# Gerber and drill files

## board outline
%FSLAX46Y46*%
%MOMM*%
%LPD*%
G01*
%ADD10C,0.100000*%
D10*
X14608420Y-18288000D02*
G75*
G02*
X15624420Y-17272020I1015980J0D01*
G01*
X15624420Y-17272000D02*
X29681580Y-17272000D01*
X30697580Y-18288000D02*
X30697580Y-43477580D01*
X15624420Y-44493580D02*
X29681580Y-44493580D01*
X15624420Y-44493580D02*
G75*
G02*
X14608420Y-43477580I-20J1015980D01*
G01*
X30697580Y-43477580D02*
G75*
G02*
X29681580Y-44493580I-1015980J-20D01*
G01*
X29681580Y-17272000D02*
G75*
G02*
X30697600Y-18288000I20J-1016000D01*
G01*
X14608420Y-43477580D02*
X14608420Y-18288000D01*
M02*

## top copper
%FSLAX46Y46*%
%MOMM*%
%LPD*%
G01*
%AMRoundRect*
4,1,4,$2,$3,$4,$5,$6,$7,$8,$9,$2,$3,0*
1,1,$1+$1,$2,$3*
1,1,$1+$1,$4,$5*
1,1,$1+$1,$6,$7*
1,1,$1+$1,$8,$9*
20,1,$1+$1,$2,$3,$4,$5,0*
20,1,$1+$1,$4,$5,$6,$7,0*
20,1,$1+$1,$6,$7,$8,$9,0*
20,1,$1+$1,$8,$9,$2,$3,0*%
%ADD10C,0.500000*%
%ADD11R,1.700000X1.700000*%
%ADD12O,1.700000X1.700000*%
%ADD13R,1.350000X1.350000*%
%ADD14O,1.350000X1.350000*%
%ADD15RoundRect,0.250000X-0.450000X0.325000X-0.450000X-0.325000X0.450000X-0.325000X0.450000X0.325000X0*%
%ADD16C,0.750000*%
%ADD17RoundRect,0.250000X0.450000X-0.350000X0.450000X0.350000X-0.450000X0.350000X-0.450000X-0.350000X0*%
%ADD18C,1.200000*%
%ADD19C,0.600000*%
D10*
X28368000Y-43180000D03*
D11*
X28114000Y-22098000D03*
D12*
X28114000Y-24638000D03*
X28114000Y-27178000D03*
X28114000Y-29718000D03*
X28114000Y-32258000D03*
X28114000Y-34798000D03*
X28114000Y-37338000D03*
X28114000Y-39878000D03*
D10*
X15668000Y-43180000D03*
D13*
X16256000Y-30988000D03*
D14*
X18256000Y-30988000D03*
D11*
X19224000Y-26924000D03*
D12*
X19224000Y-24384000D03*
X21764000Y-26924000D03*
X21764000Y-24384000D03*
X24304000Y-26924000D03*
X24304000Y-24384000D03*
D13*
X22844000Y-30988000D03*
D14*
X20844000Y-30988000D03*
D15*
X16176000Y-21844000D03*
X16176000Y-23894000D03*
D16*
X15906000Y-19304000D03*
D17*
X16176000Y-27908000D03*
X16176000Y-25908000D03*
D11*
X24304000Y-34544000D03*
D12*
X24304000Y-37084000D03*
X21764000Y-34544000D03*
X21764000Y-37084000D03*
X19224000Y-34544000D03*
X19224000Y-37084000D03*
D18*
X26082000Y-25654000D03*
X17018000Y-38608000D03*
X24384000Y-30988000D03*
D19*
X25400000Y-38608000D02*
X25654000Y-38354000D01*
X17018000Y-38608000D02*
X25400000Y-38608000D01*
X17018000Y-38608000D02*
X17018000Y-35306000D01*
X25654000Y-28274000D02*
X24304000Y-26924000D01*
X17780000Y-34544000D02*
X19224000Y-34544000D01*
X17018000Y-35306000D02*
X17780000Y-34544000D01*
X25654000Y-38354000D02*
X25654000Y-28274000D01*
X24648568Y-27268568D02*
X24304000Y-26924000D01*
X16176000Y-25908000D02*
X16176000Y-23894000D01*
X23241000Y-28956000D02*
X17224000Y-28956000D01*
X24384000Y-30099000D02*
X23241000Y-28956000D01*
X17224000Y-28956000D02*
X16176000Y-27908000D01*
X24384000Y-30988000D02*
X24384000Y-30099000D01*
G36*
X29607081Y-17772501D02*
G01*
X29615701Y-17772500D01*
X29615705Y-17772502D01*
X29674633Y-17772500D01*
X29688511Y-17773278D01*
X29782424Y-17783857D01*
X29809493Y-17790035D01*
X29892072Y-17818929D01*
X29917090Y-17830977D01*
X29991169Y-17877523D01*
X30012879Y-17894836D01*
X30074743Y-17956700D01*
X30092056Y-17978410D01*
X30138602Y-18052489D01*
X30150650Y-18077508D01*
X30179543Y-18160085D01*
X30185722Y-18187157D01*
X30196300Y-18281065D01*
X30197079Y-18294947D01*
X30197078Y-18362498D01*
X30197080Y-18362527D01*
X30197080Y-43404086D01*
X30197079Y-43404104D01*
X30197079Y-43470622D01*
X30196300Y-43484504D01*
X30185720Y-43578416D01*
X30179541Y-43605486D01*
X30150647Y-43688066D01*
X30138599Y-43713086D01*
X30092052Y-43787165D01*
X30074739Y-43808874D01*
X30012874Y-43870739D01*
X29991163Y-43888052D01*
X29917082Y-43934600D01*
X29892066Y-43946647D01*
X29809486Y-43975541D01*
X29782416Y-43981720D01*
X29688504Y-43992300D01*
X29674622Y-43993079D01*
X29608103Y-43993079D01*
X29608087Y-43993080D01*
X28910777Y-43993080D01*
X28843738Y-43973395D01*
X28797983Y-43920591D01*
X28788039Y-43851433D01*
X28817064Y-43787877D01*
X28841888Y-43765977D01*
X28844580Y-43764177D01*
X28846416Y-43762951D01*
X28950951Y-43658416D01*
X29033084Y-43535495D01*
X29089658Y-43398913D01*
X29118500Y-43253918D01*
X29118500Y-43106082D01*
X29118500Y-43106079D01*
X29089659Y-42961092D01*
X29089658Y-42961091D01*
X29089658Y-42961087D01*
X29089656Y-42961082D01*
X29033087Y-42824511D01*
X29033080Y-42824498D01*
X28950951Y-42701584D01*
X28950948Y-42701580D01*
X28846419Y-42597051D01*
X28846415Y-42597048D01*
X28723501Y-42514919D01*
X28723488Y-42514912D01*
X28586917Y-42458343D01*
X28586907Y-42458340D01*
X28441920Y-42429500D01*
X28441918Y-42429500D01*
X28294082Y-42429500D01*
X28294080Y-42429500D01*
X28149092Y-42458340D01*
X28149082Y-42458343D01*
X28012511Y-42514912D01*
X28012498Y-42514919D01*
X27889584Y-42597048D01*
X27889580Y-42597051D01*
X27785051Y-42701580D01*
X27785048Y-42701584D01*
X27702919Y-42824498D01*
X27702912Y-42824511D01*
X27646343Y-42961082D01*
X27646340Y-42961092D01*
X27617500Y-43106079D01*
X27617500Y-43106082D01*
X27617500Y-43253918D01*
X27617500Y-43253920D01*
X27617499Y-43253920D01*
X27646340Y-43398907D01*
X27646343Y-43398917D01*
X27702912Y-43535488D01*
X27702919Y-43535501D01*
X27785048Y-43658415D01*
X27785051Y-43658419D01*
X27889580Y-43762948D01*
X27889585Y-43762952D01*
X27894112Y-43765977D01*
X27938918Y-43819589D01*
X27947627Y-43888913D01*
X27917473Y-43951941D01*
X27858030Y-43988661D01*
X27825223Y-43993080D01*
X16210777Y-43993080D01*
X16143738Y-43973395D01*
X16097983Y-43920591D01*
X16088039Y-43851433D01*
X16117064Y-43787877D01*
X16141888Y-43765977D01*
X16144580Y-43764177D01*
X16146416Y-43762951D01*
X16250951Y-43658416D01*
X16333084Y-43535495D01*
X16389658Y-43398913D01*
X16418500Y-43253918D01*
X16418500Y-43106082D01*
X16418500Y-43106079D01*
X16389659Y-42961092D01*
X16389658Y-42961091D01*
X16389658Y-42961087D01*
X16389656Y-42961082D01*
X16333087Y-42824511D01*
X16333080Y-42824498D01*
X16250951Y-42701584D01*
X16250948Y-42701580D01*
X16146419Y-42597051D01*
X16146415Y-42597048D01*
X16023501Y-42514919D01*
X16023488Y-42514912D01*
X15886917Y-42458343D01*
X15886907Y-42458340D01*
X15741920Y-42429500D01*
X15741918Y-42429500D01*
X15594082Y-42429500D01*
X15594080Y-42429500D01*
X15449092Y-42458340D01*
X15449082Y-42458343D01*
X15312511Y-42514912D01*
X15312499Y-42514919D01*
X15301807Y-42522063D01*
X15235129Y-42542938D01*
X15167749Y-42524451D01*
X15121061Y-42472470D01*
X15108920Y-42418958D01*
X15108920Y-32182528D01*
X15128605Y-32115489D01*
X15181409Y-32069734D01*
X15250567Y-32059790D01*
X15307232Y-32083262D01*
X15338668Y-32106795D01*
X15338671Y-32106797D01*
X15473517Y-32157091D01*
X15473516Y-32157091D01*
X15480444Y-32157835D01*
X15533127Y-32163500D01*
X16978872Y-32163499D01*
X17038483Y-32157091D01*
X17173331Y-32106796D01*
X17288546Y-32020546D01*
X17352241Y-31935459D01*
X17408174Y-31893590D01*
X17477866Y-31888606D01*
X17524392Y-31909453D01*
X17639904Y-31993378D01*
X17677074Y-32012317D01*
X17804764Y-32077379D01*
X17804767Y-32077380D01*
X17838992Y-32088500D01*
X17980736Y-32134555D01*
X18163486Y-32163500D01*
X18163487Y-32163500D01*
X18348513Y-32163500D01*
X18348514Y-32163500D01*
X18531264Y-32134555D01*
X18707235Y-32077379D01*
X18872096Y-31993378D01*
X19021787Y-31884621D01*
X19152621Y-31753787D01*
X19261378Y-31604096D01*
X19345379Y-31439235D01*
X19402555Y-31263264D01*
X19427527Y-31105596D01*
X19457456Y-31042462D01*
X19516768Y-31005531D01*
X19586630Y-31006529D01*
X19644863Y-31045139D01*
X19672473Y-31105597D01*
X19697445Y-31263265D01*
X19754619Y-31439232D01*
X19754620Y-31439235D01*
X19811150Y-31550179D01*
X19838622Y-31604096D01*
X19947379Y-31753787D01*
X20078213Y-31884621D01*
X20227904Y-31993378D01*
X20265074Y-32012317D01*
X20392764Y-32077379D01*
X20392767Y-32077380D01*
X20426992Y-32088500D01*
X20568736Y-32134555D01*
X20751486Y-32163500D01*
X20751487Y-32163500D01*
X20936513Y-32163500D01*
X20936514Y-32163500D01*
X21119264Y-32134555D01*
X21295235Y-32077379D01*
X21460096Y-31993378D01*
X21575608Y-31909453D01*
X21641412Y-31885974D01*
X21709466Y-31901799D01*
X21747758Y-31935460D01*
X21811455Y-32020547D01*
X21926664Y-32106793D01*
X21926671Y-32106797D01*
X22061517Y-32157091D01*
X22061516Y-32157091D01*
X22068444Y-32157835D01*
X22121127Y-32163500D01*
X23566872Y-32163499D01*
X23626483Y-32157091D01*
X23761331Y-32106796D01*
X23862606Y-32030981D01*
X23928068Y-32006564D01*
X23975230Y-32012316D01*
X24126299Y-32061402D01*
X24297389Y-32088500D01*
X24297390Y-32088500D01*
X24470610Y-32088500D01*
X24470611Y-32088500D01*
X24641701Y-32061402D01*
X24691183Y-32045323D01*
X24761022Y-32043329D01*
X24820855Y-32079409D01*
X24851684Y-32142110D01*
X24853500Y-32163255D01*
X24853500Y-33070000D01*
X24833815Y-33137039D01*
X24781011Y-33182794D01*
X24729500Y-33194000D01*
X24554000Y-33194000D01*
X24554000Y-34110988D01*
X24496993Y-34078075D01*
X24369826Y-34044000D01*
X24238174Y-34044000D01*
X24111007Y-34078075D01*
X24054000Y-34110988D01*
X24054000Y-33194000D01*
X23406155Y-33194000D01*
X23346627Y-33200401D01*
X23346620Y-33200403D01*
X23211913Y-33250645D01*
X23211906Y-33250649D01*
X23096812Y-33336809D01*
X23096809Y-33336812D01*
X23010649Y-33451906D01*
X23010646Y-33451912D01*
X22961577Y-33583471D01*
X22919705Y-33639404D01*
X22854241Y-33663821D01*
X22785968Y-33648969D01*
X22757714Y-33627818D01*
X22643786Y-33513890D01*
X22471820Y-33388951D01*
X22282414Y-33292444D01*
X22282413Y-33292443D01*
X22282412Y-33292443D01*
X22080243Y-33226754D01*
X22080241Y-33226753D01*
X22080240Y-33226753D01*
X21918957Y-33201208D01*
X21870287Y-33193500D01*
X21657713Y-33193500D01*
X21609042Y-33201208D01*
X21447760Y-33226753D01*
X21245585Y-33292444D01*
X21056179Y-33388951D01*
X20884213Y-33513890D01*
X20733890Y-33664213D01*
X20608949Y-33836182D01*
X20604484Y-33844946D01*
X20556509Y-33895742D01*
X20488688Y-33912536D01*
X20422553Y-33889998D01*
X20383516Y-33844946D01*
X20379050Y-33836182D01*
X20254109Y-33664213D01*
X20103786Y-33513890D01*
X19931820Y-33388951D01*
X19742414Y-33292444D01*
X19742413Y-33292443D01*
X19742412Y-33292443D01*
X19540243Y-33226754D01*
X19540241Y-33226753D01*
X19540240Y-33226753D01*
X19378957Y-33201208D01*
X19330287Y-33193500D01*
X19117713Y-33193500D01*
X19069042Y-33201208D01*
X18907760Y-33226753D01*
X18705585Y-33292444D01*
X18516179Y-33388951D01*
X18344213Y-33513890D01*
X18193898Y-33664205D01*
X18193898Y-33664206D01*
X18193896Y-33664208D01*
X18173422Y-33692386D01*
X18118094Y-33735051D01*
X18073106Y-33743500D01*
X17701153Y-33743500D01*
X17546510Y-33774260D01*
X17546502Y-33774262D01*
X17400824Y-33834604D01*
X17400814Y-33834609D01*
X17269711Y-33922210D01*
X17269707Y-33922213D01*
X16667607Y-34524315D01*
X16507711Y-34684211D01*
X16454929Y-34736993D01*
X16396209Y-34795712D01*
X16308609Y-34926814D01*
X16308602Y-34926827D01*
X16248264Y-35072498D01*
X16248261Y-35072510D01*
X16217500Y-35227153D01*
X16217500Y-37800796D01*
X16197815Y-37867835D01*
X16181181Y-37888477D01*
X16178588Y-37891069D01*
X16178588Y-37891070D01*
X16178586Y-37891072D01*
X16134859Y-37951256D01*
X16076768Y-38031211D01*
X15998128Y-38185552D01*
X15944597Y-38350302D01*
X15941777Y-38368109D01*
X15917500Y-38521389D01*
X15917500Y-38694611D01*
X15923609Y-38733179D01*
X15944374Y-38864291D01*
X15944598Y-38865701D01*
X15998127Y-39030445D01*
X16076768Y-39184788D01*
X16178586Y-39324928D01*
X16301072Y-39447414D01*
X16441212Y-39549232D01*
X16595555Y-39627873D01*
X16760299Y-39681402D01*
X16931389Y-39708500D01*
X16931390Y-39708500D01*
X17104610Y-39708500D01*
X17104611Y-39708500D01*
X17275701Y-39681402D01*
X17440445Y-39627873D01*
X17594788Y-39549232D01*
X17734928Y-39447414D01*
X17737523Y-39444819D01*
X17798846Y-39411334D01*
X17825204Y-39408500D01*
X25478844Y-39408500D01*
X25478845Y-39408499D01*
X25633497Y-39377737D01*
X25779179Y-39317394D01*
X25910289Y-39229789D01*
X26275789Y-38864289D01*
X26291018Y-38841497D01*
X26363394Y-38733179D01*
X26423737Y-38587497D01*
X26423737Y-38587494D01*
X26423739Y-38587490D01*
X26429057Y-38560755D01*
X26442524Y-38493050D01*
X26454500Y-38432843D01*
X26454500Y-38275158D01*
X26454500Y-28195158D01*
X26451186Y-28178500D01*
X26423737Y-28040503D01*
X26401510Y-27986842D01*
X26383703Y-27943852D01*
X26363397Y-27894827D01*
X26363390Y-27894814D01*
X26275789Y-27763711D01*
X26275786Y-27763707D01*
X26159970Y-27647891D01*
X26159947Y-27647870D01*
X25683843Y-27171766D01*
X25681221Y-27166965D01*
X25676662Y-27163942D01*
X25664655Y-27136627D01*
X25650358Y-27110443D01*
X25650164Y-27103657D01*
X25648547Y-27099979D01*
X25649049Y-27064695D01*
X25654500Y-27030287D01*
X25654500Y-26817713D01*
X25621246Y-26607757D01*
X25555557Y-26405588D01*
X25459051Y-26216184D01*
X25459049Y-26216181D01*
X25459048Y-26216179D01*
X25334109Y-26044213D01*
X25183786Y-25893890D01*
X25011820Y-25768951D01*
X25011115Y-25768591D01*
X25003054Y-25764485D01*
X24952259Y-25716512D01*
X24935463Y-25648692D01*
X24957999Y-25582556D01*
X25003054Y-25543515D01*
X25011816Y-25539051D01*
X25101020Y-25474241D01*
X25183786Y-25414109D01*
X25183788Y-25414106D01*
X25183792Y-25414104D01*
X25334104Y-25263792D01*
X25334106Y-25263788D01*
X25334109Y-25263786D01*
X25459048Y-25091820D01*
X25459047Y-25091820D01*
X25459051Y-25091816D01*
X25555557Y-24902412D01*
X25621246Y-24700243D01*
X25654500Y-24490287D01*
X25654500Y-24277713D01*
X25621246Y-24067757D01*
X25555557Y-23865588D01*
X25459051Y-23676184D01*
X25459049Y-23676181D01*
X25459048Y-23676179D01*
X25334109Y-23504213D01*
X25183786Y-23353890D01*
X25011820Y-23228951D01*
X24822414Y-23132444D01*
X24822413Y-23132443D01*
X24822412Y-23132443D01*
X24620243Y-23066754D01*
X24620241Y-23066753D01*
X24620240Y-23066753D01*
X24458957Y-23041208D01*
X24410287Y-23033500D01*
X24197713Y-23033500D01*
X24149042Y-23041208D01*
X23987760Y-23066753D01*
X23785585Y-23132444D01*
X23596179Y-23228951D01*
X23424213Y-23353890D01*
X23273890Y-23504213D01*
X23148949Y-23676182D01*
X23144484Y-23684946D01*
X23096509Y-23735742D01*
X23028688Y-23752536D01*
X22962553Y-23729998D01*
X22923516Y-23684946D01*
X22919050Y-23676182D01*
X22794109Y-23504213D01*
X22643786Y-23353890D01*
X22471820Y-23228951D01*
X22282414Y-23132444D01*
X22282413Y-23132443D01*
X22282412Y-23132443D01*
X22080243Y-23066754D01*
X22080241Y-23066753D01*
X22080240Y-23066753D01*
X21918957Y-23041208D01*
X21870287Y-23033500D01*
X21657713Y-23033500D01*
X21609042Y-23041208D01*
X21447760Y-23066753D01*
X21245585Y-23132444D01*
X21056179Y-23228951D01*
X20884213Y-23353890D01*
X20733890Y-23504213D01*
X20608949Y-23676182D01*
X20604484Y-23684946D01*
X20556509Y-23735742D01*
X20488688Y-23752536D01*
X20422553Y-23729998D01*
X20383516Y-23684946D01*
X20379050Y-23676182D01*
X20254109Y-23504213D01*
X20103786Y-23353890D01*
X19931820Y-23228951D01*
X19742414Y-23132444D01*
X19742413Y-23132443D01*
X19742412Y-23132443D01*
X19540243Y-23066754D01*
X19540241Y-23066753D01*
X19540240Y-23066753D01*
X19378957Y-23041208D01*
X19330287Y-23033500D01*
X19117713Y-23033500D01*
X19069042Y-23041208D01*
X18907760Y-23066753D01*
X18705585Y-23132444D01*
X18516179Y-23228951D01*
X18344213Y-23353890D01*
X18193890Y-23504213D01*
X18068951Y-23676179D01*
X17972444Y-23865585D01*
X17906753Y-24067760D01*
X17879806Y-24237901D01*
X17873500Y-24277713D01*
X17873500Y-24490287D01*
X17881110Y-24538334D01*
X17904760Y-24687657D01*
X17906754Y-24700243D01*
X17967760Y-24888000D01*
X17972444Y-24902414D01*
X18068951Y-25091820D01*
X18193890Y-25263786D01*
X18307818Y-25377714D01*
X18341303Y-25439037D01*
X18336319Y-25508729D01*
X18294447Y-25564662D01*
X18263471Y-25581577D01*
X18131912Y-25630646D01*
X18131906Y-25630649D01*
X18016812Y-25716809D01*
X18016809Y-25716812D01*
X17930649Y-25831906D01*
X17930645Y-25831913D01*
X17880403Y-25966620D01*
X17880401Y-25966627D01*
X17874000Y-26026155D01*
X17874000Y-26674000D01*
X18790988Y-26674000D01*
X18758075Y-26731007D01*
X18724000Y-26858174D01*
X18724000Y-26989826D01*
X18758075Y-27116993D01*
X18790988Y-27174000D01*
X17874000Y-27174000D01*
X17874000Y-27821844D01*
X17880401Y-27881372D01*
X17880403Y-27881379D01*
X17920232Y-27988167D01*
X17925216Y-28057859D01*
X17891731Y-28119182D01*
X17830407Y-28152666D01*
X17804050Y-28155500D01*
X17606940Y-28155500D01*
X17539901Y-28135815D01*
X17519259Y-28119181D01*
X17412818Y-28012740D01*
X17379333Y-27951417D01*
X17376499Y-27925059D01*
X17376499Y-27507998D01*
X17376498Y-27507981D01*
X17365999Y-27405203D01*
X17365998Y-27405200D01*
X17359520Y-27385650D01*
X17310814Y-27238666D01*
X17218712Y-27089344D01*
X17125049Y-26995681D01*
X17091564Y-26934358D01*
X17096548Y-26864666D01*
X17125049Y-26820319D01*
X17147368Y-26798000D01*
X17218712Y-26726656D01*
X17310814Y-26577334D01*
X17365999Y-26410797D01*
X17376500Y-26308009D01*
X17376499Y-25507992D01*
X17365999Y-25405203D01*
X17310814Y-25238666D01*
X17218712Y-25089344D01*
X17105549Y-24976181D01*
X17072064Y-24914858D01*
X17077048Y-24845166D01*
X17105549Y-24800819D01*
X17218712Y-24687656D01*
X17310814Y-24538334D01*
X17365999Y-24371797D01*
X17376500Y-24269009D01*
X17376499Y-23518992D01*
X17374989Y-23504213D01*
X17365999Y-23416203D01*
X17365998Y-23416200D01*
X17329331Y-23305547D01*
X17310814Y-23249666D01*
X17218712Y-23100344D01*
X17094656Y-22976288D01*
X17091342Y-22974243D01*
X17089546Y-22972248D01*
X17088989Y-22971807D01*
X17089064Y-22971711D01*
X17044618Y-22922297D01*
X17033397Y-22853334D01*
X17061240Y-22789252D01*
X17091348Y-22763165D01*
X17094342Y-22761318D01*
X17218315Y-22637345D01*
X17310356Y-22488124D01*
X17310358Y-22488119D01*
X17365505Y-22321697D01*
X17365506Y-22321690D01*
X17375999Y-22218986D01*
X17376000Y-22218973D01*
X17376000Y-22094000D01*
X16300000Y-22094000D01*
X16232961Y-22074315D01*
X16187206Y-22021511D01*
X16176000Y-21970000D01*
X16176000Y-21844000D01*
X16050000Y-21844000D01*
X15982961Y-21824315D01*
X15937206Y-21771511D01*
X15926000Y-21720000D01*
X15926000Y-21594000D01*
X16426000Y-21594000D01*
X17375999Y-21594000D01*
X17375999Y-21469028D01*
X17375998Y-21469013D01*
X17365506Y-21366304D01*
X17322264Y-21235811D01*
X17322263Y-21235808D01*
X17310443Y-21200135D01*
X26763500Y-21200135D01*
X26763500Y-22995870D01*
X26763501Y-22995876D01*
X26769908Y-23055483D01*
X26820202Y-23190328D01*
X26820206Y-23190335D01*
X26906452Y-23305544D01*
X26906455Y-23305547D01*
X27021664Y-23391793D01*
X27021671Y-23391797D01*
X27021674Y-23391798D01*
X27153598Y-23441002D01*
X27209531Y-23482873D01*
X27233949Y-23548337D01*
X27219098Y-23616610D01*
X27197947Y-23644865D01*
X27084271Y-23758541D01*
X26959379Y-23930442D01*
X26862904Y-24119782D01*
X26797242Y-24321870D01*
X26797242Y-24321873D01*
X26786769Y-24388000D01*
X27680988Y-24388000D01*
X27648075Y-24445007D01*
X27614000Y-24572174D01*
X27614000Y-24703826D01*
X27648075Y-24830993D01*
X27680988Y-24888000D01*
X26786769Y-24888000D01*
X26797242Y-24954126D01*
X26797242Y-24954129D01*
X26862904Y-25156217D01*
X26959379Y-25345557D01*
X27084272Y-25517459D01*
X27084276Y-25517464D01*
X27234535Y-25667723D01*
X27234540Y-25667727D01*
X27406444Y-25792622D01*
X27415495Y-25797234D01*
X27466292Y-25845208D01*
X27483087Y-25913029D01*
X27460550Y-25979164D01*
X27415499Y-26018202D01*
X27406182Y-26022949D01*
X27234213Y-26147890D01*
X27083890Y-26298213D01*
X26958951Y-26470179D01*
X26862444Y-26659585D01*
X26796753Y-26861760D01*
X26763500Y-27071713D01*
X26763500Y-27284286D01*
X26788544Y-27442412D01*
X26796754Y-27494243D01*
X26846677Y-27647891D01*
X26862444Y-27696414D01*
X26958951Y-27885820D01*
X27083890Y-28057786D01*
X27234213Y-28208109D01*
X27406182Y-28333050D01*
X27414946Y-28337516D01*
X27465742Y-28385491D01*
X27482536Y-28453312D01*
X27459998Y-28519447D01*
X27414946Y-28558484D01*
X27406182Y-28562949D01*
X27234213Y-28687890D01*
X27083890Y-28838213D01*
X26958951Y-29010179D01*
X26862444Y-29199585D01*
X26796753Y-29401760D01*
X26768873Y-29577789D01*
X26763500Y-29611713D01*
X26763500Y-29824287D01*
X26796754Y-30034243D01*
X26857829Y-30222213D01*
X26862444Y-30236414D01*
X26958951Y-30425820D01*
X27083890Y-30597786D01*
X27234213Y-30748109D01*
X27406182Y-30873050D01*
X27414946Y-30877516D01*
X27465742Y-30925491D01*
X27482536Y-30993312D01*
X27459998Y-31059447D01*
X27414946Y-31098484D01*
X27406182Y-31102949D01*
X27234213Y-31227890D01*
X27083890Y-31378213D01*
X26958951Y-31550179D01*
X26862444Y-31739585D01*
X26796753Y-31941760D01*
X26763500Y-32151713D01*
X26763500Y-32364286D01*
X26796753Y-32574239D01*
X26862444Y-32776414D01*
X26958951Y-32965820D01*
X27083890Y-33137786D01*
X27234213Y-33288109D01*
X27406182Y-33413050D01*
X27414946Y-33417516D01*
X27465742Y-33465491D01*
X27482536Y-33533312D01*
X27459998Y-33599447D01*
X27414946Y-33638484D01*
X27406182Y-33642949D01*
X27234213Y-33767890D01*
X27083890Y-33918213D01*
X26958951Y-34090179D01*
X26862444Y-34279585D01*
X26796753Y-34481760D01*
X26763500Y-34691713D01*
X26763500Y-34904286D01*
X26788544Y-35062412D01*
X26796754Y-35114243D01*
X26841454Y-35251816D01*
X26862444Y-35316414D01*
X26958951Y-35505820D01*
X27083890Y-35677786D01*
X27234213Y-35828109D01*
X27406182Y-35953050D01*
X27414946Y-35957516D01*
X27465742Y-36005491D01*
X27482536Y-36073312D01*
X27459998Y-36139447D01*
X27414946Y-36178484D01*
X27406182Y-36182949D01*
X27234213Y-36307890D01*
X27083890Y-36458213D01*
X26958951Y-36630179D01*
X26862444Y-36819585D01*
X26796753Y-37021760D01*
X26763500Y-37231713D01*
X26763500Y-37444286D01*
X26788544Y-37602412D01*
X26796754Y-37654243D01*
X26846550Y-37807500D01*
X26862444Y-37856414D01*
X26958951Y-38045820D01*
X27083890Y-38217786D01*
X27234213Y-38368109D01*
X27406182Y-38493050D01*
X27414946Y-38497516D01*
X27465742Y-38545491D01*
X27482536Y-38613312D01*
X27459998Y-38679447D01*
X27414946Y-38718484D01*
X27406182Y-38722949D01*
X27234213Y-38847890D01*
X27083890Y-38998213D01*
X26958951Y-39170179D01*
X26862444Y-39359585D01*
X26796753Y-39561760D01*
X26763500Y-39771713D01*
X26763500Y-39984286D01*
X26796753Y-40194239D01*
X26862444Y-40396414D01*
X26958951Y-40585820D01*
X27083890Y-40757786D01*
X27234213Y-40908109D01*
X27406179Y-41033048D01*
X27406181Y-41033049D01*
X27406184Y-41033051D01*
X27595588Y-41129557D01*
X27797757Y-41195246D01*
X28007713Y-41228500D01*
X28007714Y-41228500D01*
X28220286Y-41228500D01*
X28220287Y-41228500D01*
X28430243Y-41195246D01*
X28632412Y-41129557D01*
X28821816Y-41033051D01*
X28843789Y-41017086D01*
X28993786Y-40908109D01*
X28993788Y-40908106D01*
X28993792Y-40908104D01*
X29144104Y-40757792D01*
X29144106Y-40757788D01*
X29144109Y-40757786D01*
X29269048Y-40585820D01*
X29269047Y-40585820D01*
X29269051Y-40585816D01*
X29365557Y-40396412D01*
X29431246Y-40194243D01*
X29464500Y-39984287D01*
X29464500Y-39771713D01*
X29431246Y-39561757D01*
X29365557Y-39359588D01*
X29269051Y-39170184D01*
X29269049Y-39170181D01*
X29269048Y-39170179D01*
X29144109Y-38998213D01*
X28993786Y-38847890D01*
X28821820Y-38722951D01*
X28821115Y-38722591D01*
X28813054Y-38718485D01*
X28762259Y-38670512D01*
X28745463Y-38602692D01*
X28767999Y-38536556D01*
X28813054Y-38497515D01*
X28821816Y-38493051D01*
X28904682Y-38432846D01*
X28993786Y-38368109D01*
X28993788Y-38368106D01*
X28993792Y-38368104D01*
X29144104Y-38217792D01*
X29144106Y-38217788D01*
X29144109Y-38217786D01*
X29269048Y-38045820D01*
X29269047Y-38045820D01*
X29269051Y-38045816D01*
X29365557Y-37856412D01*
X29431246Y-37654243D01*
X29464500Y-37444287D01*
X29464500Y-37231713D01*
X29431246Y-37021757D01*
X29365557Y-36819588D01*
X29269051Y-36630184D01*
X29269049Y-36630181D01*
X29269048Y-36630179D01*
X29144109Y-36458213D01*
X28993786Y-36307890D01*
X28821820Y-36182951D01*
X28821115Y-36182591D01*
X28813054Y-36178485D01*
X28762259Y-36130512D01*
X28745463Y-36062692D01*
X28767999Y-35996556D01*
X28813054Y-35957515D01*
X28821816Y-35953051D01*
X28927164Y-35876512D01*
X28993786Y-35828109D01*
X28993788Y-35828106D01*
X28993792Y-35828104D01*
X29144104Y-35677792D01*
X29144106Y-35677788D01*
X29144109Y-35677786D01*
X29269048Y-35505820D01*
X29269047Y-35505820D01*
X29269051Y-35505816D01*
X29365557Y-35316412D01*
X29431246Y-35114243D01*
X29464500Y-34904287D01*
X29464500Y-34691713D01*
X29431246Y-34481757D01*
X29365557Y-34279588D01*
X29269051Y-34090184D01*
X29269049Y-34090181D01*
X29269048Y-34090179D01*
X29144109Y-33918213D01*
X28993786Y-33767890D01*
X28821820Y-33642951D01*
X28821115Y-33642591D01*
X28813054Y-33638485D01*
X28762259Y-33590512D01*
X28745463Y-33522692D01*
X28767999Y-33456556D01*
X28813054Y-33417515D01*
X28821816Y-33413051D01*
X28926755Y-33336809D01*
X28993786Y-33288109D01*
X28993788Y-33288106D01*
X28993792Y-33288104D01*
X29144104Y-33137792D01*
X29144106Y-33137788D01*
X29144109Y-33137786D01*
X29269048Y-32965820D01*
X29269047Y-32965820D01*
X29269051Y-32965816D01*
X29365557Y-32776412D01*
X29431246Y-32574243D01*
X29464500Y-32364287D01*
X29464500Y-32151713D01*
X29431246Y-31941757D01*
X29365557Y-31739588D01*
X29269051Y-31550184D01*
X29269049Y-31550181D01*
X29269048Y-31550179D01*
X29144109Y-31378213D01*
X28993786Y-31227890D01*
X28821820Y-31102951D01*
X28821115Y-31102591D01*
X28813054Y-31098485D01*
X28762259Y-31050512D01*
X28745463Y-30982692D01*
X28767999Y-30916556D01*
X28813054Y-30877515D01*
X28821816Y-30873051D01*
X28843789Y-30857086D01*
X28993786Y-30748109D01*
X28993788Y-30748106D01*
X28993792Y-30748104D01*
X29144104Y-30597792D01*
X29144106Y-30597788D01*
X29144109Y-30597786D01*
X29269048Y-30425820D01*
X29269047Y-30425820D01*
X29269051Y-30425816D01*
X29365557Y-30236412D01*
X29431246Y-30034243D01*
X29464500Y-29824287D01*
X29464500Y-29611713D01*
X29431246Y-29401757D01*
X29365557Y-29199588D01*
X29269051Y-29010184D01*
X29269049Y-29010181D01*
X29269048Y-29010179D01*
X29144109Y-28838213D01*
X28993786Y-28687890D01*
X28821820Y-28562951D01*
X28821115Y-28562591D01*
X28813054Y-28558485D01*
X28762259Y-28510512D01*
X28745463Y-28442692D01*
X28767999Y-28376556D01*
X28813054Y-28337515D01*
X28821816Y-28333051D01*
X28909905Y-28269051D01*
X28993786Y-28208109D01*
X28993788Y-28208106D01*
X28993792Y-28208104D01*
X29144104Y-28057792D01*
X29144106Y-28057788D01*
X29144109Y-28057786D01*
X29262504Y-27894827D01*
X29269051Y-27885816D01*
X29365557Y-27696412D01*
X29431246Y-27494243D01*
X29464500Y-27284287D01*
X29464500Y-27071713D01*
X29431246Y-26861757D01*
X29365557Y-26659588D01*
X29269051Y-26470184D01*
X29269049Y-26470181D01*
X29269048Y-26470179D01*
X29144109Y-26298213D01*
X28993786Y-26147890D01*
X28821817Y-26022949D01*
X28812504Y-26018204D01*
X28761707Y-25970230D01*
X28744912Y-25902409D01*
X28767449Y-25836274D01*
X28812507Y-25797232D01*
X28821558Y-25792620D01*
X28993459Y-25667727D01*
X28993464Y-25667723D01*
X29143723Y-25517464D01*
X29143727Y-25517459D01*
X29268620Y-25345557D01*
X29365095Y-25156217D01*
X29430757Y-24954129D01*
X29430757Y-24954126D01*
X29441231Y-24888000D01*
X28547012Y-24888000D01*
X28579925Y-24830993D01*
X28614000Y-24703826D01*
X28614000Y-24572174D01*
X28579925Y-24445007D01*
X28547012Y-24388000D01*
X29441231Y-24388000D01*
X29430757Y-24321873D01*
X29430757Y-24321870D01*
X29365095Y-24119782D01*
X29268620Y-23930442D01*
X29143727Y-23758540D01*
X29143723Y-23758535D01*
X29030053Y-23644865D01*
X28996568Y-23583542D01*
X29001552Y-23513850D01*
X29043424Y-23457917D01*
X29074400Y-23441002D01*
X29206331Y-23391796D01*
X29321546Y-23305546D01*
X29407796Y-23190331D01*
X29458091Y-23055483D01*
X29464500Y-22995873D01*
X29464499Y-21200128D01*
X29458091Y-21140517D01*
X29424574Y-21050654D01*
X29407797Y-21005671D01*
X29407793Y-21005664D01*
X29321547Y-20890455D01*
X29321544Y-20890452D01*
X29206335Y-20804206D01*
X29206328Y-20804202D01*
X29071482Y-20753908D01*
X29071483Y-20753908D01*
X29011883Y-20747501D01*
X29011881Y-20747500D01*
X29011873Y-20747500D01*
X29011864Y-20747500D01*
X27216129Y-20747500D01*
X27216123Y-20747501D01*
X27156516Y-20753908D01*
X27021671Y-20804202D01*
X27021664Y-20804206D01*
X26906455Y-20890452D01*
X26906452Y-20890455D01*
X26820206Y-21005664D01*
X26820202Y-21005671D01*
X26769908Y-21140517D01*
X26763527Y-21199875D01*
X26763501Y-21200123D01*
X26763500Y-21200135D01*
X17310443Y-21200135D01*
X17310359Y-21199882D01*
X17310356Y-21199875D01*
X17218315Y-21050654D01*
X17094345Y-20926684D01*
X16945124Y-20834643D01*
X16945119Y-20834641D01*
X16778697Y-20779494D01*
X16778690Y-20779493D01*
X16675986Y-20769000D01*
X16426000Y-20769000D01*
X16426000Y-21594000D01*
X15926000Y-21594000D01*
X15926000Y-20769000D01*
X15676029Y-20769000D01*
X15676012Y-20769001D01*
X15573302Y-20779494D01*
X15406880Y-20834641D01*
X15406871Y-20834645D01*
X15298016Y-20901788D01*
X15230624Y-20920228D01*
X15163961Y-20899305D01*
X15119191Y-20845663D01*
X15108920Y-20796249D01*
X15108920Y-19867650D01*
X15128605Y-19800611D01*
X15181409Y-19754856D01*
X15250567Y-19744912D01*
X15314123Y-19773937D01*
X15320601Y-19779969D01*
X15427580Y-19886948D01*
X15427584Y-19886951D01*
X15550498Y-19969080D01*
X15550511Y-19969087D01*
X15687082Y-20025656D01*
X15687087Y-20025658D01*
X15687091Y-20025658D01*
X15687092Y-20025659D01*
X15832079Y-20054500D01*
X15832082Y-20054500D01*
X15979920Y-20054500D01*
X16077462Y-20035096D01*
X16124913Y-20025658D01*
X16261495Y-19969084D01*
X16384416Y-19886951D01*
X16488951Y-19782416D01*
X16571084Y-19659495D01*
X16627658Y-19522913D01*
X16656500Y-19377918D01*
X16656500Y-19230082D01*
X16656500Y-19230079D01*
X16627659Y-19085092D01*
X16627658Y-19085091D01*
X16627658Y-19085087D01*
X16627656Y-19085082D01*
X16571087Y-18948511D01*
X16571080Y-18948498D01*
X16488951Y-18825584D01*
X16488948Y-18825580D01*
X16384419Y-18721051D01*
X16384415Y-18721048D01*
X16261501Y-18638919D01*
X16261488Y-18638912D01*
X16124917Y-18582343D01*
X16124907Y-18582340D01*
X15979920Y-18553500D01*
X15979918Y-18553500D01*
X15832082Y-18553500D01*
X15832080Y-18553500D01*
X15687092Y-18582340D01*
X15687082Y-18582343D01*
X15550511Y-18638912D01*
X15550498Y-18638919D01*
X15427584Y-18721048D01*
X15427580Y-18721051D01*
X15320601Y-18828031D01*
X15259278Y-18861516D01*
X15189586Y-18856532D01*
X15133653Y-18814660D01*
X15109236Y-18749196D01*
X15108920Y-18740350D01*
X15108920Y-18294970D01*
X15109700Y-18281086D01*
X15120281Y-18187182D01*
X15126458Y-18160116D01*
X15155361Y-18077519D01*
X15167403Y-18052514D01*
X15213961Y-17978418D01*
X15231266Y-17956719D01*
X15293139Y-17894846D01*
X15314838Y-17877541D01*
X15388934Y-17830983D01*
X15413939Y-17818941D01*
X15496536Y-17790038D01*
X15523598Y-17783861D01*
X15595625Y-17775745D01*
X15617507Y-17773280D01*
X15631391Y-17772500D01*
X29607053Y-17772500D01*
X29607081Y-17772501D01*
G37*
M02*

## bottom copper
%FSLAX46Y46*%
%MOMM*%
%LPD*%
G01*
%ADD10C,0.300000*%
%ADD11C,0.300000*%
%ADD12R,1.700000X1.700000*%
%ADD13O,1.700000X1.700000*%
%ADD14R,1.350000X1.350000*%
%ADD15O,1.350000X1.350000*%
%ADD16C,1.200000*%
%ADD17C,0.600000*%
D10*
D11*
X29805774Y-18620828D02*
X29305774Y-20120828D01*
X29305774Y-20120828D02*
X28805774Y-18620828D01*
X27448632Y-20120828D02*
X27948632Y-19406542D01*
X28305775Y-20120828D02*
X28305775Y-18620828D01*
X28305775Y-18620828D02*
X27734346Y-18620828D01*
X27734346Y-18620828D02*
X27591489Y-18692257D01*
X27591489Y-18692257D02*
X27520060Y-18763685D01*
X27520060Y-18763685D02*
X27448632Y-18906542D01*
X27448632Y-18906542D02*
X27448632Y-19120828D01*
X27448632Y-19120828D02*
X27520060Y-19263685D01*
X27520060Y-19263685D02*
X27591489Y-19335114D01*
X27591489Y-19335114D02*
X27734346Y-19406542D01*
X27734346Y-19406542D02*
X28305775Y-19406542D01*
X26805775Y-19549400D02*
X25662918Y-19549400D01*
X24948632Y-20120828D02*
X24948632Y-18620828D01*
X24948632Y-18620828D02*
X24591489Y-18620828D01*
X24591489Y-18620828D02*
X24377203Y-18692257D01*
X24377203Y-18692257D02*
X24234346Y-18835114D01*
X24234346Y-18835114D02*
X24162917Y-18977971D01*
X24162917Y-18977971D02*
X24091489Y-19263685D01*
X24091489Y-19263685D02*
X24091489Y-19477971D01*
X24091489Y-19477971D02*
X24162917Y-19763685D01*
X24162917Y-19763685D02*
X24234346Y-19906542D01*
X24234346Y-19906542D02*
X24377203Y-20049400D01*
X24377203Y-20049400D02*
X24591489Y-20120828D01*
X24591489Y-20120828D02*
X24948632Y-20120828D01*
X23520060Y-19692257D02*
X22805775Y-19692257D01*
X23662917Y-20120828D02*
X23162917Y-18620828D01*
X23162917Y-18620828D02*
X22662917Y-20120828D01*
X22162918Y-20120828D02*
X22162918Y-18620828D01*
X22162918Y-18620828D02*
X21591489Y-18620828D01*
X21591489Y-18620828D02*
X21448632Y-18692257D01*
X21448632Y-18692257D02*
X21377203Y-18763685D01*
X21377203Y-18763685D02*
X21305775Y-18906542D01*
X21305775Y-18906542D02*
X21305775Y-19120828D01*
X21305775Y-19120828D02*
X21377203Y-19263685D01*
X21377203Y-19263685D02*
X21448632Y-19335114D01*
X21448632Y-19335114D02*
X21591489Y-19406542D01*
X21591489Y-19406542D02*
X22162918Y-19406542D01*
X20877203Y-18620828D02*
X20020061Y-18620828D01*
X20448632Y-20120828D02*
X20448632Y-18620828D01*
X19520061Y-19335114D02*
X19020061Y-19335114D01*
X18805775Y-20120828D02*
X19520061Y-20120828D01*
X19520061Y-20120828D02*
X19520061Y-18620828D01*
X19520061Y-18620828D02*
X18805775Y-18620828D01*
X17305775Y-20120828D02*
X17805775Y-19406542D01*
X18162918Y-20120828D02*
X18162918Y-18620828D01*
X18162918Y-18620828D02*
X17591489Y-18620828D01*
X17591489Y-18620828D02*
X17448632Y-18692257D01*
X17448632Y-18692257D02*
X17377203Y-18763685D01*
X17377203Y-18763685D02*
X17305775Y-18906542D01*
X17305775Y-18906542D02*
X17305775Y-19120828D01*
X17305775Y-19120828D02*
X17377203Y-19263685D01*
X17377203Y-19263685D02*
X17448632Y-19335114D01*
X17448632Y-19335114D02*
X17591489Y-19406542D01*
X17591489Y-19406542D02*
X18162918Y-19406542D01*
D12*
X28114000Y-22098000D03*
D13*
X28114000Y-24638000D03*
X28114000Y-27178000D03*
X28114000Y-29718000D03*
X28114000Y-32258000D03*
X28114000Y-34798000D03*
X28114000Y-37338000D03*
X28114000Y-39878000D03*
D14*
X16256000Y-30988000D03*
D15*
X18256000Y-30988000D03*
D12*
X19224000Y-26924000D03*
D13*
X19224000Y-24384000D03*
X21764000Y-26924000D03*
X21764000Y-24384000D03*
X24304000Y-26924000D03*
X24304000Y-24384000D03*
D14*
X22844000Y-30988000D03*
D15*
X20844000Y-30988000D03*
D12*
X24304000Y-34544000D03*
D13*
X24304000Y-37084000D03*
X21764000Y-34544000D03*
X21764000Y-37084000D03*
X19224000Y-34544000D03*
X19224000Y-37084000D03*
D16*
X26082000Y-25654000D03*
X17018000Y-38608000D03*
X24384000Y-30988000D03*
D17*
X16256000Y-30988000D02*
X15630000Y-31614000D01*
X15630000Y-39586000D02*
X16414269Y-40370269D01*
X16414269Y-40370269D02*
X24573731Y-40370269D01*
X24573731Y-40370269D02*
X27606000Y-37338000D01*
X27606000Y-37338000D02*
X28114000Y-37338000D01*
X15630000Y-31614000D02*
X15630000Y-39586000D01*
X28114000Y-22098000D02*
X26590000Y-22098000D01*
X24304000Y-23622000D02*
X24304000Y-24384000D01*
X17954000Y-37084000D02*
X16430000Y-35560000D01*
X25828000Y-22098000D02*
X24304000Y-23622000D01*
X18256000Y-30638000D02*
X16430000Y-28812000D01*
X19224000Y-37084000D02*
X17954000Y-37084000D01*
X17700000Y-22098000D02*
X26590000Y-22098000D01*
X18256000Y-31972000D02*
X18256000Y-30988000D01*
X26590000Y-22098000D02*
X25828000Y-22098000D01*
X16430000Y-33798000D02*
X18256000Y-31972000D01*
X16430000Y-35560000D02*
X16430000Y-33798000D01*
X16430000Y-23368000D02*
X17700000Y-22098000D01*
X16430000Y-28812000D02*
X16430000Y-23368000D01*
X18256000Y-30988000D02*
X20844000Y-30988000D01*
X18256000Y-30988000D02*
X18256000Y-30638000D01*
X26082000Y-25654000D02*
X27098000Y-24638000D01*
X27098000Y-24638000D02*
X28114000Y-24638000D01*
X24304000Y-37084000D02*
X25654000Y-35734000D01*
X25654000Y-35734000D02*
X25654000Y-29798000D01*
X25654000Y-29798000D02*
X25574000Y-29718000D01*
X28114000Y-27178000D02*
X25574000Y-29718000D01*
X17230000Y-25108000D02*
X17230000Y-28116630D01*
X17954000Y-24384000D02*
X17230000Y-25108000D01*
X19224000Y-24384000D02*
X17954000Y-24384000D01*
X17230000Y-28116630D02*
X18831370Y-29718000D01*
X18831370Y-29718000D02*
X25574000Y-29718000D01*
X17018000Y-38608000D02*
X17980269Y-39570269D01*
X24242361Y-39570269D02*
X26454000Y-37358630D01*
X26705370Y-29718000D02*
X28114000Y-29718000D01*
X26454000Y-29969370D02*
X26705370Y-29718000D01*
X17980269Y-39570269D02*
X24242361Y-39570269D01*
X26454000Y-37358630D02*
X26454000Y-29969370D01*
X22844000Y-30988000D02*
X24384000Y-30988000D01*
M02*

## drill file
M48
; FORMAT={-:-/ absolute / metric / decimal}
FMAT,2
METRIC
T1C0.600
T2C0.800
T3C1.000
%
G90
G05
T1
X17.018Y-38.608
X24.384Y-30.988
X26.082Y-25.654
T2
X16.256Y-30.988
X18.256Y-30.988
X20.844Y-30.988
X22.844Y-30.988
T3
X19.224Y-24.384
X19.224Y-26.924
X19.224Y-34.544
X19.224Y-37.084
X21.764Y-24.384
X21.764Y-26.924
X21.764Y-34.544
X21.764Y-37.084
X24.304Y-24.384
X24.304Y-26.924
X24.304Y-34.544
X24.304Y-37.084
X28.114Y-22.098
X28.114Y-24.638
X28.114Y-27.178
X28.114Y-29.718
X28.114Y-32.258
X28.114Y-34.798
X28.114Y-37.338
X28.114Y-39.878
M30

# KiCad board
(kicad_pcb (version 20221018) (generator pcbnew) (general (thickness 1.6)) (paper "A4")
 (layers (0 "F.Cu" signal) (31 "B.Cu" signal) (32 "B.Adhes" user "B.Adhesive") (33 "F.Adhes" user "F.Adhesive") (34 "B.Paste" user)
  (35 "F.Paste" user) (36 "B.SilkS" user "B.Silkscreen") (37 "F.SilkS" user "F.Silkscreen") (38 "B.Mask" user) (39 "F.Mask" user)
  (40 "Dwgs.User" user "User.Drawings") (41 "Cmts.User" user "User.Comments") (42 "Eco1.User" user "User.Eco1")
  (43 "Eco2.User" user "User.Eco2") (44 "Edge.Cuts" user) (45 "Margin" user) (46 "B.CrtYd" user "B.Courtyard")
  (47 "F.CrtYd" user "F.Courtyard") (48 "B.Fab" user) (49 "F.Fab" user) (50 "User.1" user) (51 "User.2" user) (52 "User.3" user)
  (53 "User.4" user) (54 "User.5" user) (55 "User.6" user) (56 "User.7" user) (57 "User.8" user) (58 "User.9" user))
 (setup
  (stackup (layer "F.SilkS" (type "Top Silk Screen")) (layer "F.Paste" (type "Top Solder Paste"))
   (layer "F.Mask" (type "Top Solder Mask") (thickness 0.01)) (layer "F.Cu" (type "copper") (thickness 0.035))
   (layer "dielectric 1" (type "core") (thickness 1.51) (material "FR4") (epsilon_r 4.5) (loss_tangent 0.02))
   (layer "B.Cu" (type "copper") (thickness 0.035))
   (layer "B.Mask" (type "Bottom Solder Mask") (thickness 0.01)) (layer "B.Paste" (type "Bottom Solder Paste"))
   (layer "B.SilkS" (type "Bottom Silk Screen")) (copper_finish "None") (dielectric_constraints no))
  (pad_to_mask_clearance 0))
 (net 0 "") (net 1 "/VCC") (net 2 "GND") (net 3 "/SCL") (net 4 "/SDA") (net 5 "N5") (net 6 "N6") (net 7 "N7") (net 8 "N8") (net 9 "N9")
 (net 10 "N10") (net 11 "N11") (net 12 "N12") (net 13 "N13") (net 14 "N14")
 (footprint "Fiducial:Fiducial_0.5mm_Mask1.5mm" (layer "F.Cu") (at 28.368 43.18)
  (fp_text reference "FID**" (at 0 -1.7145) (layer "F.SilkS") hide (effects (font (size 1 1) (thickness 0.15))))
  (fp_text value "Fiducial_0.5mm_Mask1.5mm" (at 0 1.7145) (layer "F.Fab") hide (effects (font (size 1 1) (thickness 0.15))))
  (pad "" smd circle (at 0 0) (size 0.5 0.5) (layers "F.Cu" "F.Mask" "Eco1.User") (solder_mask_margin 0.5) (clearance 0.5)))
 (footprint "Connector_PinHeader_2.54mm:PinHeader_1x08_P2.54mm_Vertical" (layer "F.Cu") (at 28.114 22.098)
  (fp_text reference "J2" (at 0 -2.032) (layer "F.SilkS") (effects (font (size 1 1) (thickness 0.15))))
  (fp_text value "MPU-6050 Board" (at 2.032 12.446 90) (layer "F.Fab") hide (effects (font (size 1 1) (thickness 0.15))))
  (pad "1" thru_hole rect (at 0 0) (size 1.7 1.7) (drill 1) (layers "*.Cu" "*.Mask") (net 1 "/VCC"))
  (pad "2" thru_hole oval (at 0 2.54) (size 1.7 1.7) (drill 1) (layers "*.Cu" "*.Mask") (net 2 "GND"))
  (pad "3" thru_hole oval (at 0 5.08) (size 1.7 1.7) (drill 1) (layers "*.Cu" "*.Mask") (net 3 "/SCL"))
  (pad "4" thru_hole oval (at 0 7.62) (size 1.7 1.7) (drill 1) (layers "*.Cu" "*.Mask") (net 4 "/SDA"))
  (pad "5" thru_hole oval (at 0 10.16) (size 1.7 1.7) (drill 1) (layers "*.Cu" "*.Mask") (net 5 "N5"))
  (pad "6" thru_hole oval (at 0 12.7) (size 1.7 1.7) (drill 1) (layers "*.Cu" "*.Mask") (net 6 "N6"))
  (pad "7" thru_hole oval (at 0 15.24) (size 1.7 1.7) (drill 1) (layers "*.Cu" "*.Mask") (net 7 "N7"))
  (pad "8" thru_hole oval (at 0 17.78) (size 1.7 1.7) (drill 1) (layers "*.Cu" "*.Mask") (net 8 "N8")))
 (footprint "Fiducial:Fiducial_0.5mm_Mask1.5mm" (layer "F.Cu") (at 15.668 43.18)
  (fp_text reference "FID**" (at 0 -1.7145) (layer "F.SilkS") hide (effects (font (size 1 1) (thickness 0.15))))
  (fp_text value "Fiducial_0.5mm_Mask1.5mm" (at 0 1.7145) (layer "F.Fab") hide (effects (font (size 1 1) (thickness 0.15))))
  (pad "" smd circle (at 0 0) (size 0.5 0.5) (layers "F.Cu" "F.Mask" "Eco1.User") (solder_mask_margin 0.5) (clearance 0.5)))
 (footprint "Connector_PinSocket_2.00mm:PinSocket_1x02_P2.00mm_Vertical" (layer "F.Cu") (at 16.256 30.988 90)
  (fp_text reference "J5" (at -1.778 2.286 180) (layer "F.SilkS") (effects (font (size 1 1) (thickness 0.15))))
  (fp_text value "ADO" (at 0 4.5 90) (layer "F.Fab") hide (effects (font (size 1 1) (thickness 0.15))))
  (pad "1" thru_hole rect (at 0 0 90) (size 1.35 1.35) (drill 0.8) (layers "*.Cu" "*.Mask") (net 7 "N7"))
  (pad "2" thru_hole oval (at 0 2 90) (size 1.35 1.35) (drill 0.8) (layers "*.Cu" "*.Mask") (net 1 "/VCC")))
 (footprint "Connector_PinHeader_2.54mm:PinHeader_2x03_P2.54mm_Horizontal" (layer "F.Cu") (at 19.224 26.924 90)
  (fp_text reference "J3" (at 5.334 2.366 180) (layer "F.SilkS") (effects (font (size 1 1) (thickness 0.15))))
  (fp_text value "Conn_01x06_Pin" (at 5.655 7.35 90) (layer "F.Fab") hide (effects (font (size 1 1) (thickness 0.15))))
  (pad "1" thru_hole rect (at 0 0 90) (size 1.7 1.7) (drill 1) (layers "*.Cu" "*.Mask") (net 2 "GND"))
  (pad "2" thru_hole oval (at 2.54 0 90) (size 1.7 1.7) (drill 1) (layers "*.Cu" "*.Mask") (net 3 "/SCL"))
  (pad "3" thru_hole oval (at 0 2.54 90) (size 1.7 1.7) (drill 1) (layers "*.Cu" "*.Mask") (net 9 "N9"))
  (pad "4" thru_hole oval (at 2.54 2.54 90) (size 1.7 1.7) (drill 1) (layers "*.Cu" "*.Mask") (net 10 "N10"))
  (pad "5" thru_hole oval (at 0 5.08 90) (size 1.7 1.7) (drill 1) (layers "*.Cu" "*.Mask") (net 4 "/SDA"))
  (pad "6" thru_hole oval (at 2.54 5.08 90) (size 1.7 1.7) (drill 1) (layers "*.Cu" "*.Mask") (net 1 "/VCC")))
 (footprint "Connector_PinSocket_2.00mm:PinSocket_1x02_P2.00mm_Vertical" (layer "F.Cu") (at 22.844 30.988 -90)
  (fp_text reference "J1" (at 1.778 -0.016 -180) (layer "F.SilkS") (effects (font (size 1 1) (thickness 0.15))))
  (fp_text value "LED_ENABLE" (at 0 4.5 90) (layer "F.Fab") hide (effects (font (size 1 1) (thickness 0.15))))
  (pad "1" thru_hole rect (at 0 0 270) (size 1.35 1.35) (drill 0.8) (layers "*.Cu" "*.Mask") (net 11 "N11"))
  (pad "2" thru_hole oval (at 0 2 270) (size 1.35 1.35) (drill 0.8) (layers "*.Cu" "*.Mask") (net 1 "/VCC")))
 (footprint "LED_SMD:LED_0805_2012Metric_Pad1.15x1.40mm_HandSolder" (layer "F.Cu") (at 16.176 22.869 -90)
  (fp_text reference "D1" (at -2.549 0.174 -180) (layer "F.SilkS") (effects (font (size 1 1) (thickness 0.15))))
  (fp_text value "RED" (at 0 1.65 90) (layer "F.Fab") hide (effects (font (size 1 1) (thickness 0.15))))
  (pad "1" smd roundrect (at -1.025 0 270) (size 1.15 1.4) (layers "F.Cu" "F.Paste" "F.Mask") (roundrect_rratio 0.2173913043) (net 2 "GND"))
  (pad "2" smd roundrect (at 1.025 0 270) (size 1.15 1.4) (layers "F.Cu" "F.Paste" "F.Mask") (roundrect_rratio 0.2173913043) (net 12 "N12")))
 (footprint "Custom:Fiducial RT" (layer "F.Cu") (at 15.922 19.304)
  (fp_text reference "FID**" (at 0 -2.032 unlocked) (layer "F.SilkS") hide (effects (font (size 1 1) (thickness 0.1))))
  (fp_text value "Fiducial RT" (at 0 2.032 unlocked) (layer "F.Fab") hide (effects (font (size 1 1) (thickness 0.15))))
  (pad "" smd circle (at -0.016 0) (size 0.75 0.75) (layers "F.Cu" "F.Mask" "Eco1.User") (solder_mask_margin 0.375) (clearance 0.375)))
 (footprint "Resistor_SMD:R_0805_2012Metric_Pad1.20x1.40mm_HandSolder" (layer "F.Cu") (at 16.176 26.908 90)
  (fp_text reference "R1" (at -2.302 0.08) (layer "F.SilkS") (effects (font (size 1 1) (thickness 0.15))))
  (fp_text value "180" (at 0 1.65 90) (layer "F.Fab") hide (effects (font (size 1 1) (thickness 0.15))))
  (pad "1" smd roundrect (at -1 0 90) (size 1.2 1.4) (layers "F.Cu" "F.Paste" "F.Mask") (roundrect_rratio 0.2083333333) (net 11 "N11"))
  (pad "2" smd roundrect (at 1 0 90) (size 1.2 1.4) (layers "F.Cu" "F.Paste" "F.Mask") (roundrect_rratio 0.2083333333) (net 12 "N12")))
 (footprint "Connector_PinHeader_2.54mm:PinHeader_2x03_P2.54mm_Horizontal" (layer "F.Cu") (at 24.304 34.544 -90)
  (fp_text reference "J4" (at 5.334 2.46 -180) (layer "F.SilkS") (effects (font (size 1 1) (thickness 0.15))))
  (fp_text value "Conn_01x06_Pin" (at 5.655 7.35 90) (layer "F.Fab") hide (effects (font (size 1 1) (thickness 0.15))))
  (pad "1" thru_hole rect (at 0 0 270) (size 1.7 1.7) (drill 1) (layers "*.Cu" "*.Mask") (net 2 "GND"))
  (pad "2" thru_hole oval (at 2.54 0 270) (size 1.7 1.7) (drill 1) (layers "*.Cu" "*.Mask") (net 3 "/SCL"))
  (pad "3" thru_hole oval (at 0 2.54 270) (size 1.7 1.7) (drill 1) (layers "*.Cu" "*.Mask") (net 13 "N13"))
  (pad "4" thru_hole oval (at 2.54 2.54 270) (size 1.7 1.7) (drill 1) (layers "*.Cu" "*.Mask") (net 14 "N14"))
  (pad "5" thru_hole oval (at 0 5.08 270) (size 1.7 1.7) (drill 1) (layers "*.Cu" "*.Mask") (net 4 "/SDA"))
  (pad "6" thru_hole oval (at 2.54 5.08 270) (size 1.7 1.7) (drill 1) (layers "*.Cu" "*.Mask") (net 1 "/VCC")))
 (gr_arc (start 14.60842 18.288) (mid 14.906001 17.569587) (end 15.62442 17.272) (stroke (width 0.1) (type default)) (layer "Edge.Cuts"))
 (gr_line (start 15.62442 17.272) (end 29.68158 17.272) (stroke (width 0.1) (type default)) (layer "Edge.Cuts"))
 (gr_line (start 30.69758 18.288) (end 30.69758 43.47758) (stroke (width 0.1) (type default)) (layer "Edge.Cuts"))
 (gr_line (start 15.62442 44.49358) (end 29.68158 44.49358) (stroke (width 0.1) (type default)) (layer "Edge.Cuts"))
 (gr_arc (start 15.62442 44.49358) (mid 14.905994 44.196006) (end 14.60842 43.47758) (stroke (width 0.1) (type default)) (layer "Edge.Cuts"))
 (gr_arc (start 30.69758 43.47758) (mid 30.400006 44.196006) (end 29.68158 44.49358) (stroke (width 0.1) (type default)) (layer "Edge.Cuts"))
 (gr_arc (start 29.68158 17.272) (mid 30.400013 17.569572) (end 30.69758 18.288) (stroke (width 0.1) (type default)) (layer "Edge.Cuts"))
 (gr_line (start 14.60842 43.47758) (end 14.60842 18.288) (stroke (width 0.1) (type default)) (layer "Edge.Cuts"))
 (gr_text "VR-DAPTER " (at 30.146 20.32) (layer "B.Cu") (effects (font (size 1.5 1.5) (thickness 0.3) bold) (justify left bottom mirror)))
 (segment (start 16.256 30.988) (end 15.63 31.614) (width 0.6) (layer "B.Cu") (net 7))
 (segment (start 15.63 39.586) (end 16.414269 40.370269) (width 0.6) (layer "B.Cu") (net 7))
 (segment (start 16.414269 40.370269) (end 24.573731 40.370269) (width 0.6) (layer "B.Cu") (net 7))
 (segment (start 24.573731 40.370269) (end 27.606 37.338) (width 0.6) (layer "B.Cu") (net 7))
 (segment (start 27.606 37.338) (end 28.114 37.338) (width 0.6) (layer "B.Cu") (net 7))
 (segment (start 15.63 31.614) (end 15.63 39.586) (width 0.6) (layer "B.Cu") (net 7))
 (segment (start 28.114 22.098) (end 26.59 22.098) (width 0.6) (layer "B.Cu") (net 1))
 (segment (start 24.304 23.622) (end 24.304 24.384) (width 0.6) (layer "B.Cu") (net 1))
 (segment (start 17.954 37.084) (end 16.43 35.56) (width 0.6) (layer "B.Cu") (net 1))
 (segment (start 25.828 22.098) (end 24.304 23.622) (width 0.6) (layer "B.Cu") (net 1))
 (segment (start 18.256 30.638) (end 16.43 28.812) (width 0.6) (layer "B.Cu") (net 1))
 (segment (start 19.224 37.084) (end 17.954 37.084) (width 0.6) (layer "B.Cu") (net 1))
 (segment (start 17.7 22.098) (end 26.59 22.098) (width 0.6) (layer "B.Cu") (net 1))
 (segment (start 18.256 31.972) (end 18.256 30.988) (width 0.6) (layer "B.Cu") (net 1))
 (segment (start 26.59 22.098) (end 25.828 22.098) (width 0.6) (layer "B.Cu") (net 1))
 (segment (start 16.43 33.798) (end 18.256 31.972) (width 0.6) (layer "B.Cu") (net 1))
 (segment (start 16.43 35.56) (end 16.43 33.798) (width 0.6) (layer "B.Cu") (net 1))
 (segment (start 16.43 23.368) (end 17.7 22.098) (width 0.6) (layer "B.Cu") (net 1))
 (segment (start 16.43 28.812) (end 16.43 23.368) (width 0.6) (layer "B.Cu") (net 1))
 (segment (start 18.256 30.988) (end 20.844 30.988) (width 0.6) (layer "B.Cu") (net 1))
 (segment (start 18.256 30.988) (end 18.256 30.638) (width 0.6) (layer "B.Cu") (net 1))
 (via (at 26.082 25.654) (size 1.2) (drill 0.6) (layers "F.Cu" "B.Cu") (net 2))
 (segment (start 26.082 25.654) (end 27.098 24.638) (width 0.6) (layer "B.Cu") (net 2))
 (segment (start 27.098 24.638) (end 28.114 24.638) (width 0.6) (layer "B.Cu") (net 2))
 (segment (start 24.304 37.084) (end 25.654 35.734) (width 0.6) (layer "B.Cu") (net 3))
 (segment (start 25.654 35.734) (end 25.654 29.798) (width 0.6) (layer "B.Cu") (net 3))
 (segment (start 25.654 29.798) (end 25.574 29.718) (width 0.6) (layer "B.Cu") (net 3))
 (segment (start 28.114 27.178) (end 25.574 29.718) (width 0.6) (layer "B.Cu") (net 3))
 (segment (start 17.23 25.108) (end 17.23 28.11663) (width 0.6) (layer "B.Cu") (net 3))
 (segment (start 17.954 24.384) (end 17.23 25.108) (width 0.6) (layer "B.Cu") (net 3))
 (segment (start 19.224 24.384) (end 17.954 24.384) (width 0.6) (layer "B.Cu") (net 3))
 (segment (start 17.23 28.11663) (end 18.83137 29.718) (width 0.6) (layer "B.Cu") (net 3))
 (segment (start 18.83137 29.718) (end 25.574 29.718) (width 0.6) (layer "B.Cu") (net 3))
 (segment (start 25.4 38.608) (end 25.654 38.354) (width 0.6) (layer "F.Cu") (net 4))
 (segment (start 17.018 38.608) (end 25.4 38.608) (width 0.6) (layer "F.Cu") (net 4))
 (segment (start 17.018 38.608) (end 17.018 35.306) (width 0.6) (layer "F.Cu") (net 4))
 (segment (start 25.654 28.274) (end 24.304 26.924) (width 0.6) (layer "F.Cu") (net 4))
 (segment (start 17.78 34.544) (end 19.224 34.544) (width 0.6) (layer "F.Cu") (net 4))
 (segment (start 17.018 35.306) (end 17.78 34.544) (width 0.6) (layer "F.Cu") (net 4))
 (segment (start 25.654 38.354) (end 25.654 28.274) (width 0.6) (layer "F.Cu") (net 4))
 (segment (start 24.648568 27.268568) (end 24.304 26.924) (width 0.6) (layer "F.Cu") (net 4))
 (via (at 17.018 38.608) (size 1.2) (drill 0.6) (layers "F.Cu" "B.Cu") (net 4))
 (segment (start 17.018 38.608) (end 17.980269 39.570269) (width 0.6) (layer "B.Cu") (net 4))
 (segment (start 24.242361 39.570269) (end 26.454 37.35863) (width 0.6) (layer "B.Cu") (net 4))
 (segment (start 26.70537 29.718) (end 28.114 29.718) (width 0.6) (layer "B.Cu") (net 4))
 (segment (start 26.454 29.96937) (end 26.70537 29.718) (width 0.6) (layer "B.Cu") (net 4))
 (segment (start 17.980269 39.570269) (end 24.242361 39.570269) (width 0.6) (layer "B.Cu") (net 4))
 (segment (start 26.454 37.35863) (end 26.454 29.96937) (width 0.6) (layer "B.Cu") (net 4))
 (segment (start 16.176 25.908) (end 16.176 23.894) (width 0.6) (layer "F.Cu") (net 12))
 (segment (start 23.241 28.956) (end 17.224 28.956) (width 0.6) (layer "F.Cu") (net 11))
 (segment (start 24.384 30.099) (end 23.241 28.956) (width 0.6) (layer "F.Cu") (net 11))
 (segment (start 17.224 28.956) (end 16.176 27.908) (width 0.6) (layer "F.Cu") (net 11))
 (segment (start 24.384 30.988) (end 24.384 30.099) (width 0.6) (layer "F.Cu") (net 11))
 (via (at 24.384 30.988) (size 1.2) (drill 0.6) (layers "F.Cu" "B.Cu") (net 11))
 (segment (start 22.844 30.988) (end 24.384 30.988) (width 0.6) (layer "B.Cu") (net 11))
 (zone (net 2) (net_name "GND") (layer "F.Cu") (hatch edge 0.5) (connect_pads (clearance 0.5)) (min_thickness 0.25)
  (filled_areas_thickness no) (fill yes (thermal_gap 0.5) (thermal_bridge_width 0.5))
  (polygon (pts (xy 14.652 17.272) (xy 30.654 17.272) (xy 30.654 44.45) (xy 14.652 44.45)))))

